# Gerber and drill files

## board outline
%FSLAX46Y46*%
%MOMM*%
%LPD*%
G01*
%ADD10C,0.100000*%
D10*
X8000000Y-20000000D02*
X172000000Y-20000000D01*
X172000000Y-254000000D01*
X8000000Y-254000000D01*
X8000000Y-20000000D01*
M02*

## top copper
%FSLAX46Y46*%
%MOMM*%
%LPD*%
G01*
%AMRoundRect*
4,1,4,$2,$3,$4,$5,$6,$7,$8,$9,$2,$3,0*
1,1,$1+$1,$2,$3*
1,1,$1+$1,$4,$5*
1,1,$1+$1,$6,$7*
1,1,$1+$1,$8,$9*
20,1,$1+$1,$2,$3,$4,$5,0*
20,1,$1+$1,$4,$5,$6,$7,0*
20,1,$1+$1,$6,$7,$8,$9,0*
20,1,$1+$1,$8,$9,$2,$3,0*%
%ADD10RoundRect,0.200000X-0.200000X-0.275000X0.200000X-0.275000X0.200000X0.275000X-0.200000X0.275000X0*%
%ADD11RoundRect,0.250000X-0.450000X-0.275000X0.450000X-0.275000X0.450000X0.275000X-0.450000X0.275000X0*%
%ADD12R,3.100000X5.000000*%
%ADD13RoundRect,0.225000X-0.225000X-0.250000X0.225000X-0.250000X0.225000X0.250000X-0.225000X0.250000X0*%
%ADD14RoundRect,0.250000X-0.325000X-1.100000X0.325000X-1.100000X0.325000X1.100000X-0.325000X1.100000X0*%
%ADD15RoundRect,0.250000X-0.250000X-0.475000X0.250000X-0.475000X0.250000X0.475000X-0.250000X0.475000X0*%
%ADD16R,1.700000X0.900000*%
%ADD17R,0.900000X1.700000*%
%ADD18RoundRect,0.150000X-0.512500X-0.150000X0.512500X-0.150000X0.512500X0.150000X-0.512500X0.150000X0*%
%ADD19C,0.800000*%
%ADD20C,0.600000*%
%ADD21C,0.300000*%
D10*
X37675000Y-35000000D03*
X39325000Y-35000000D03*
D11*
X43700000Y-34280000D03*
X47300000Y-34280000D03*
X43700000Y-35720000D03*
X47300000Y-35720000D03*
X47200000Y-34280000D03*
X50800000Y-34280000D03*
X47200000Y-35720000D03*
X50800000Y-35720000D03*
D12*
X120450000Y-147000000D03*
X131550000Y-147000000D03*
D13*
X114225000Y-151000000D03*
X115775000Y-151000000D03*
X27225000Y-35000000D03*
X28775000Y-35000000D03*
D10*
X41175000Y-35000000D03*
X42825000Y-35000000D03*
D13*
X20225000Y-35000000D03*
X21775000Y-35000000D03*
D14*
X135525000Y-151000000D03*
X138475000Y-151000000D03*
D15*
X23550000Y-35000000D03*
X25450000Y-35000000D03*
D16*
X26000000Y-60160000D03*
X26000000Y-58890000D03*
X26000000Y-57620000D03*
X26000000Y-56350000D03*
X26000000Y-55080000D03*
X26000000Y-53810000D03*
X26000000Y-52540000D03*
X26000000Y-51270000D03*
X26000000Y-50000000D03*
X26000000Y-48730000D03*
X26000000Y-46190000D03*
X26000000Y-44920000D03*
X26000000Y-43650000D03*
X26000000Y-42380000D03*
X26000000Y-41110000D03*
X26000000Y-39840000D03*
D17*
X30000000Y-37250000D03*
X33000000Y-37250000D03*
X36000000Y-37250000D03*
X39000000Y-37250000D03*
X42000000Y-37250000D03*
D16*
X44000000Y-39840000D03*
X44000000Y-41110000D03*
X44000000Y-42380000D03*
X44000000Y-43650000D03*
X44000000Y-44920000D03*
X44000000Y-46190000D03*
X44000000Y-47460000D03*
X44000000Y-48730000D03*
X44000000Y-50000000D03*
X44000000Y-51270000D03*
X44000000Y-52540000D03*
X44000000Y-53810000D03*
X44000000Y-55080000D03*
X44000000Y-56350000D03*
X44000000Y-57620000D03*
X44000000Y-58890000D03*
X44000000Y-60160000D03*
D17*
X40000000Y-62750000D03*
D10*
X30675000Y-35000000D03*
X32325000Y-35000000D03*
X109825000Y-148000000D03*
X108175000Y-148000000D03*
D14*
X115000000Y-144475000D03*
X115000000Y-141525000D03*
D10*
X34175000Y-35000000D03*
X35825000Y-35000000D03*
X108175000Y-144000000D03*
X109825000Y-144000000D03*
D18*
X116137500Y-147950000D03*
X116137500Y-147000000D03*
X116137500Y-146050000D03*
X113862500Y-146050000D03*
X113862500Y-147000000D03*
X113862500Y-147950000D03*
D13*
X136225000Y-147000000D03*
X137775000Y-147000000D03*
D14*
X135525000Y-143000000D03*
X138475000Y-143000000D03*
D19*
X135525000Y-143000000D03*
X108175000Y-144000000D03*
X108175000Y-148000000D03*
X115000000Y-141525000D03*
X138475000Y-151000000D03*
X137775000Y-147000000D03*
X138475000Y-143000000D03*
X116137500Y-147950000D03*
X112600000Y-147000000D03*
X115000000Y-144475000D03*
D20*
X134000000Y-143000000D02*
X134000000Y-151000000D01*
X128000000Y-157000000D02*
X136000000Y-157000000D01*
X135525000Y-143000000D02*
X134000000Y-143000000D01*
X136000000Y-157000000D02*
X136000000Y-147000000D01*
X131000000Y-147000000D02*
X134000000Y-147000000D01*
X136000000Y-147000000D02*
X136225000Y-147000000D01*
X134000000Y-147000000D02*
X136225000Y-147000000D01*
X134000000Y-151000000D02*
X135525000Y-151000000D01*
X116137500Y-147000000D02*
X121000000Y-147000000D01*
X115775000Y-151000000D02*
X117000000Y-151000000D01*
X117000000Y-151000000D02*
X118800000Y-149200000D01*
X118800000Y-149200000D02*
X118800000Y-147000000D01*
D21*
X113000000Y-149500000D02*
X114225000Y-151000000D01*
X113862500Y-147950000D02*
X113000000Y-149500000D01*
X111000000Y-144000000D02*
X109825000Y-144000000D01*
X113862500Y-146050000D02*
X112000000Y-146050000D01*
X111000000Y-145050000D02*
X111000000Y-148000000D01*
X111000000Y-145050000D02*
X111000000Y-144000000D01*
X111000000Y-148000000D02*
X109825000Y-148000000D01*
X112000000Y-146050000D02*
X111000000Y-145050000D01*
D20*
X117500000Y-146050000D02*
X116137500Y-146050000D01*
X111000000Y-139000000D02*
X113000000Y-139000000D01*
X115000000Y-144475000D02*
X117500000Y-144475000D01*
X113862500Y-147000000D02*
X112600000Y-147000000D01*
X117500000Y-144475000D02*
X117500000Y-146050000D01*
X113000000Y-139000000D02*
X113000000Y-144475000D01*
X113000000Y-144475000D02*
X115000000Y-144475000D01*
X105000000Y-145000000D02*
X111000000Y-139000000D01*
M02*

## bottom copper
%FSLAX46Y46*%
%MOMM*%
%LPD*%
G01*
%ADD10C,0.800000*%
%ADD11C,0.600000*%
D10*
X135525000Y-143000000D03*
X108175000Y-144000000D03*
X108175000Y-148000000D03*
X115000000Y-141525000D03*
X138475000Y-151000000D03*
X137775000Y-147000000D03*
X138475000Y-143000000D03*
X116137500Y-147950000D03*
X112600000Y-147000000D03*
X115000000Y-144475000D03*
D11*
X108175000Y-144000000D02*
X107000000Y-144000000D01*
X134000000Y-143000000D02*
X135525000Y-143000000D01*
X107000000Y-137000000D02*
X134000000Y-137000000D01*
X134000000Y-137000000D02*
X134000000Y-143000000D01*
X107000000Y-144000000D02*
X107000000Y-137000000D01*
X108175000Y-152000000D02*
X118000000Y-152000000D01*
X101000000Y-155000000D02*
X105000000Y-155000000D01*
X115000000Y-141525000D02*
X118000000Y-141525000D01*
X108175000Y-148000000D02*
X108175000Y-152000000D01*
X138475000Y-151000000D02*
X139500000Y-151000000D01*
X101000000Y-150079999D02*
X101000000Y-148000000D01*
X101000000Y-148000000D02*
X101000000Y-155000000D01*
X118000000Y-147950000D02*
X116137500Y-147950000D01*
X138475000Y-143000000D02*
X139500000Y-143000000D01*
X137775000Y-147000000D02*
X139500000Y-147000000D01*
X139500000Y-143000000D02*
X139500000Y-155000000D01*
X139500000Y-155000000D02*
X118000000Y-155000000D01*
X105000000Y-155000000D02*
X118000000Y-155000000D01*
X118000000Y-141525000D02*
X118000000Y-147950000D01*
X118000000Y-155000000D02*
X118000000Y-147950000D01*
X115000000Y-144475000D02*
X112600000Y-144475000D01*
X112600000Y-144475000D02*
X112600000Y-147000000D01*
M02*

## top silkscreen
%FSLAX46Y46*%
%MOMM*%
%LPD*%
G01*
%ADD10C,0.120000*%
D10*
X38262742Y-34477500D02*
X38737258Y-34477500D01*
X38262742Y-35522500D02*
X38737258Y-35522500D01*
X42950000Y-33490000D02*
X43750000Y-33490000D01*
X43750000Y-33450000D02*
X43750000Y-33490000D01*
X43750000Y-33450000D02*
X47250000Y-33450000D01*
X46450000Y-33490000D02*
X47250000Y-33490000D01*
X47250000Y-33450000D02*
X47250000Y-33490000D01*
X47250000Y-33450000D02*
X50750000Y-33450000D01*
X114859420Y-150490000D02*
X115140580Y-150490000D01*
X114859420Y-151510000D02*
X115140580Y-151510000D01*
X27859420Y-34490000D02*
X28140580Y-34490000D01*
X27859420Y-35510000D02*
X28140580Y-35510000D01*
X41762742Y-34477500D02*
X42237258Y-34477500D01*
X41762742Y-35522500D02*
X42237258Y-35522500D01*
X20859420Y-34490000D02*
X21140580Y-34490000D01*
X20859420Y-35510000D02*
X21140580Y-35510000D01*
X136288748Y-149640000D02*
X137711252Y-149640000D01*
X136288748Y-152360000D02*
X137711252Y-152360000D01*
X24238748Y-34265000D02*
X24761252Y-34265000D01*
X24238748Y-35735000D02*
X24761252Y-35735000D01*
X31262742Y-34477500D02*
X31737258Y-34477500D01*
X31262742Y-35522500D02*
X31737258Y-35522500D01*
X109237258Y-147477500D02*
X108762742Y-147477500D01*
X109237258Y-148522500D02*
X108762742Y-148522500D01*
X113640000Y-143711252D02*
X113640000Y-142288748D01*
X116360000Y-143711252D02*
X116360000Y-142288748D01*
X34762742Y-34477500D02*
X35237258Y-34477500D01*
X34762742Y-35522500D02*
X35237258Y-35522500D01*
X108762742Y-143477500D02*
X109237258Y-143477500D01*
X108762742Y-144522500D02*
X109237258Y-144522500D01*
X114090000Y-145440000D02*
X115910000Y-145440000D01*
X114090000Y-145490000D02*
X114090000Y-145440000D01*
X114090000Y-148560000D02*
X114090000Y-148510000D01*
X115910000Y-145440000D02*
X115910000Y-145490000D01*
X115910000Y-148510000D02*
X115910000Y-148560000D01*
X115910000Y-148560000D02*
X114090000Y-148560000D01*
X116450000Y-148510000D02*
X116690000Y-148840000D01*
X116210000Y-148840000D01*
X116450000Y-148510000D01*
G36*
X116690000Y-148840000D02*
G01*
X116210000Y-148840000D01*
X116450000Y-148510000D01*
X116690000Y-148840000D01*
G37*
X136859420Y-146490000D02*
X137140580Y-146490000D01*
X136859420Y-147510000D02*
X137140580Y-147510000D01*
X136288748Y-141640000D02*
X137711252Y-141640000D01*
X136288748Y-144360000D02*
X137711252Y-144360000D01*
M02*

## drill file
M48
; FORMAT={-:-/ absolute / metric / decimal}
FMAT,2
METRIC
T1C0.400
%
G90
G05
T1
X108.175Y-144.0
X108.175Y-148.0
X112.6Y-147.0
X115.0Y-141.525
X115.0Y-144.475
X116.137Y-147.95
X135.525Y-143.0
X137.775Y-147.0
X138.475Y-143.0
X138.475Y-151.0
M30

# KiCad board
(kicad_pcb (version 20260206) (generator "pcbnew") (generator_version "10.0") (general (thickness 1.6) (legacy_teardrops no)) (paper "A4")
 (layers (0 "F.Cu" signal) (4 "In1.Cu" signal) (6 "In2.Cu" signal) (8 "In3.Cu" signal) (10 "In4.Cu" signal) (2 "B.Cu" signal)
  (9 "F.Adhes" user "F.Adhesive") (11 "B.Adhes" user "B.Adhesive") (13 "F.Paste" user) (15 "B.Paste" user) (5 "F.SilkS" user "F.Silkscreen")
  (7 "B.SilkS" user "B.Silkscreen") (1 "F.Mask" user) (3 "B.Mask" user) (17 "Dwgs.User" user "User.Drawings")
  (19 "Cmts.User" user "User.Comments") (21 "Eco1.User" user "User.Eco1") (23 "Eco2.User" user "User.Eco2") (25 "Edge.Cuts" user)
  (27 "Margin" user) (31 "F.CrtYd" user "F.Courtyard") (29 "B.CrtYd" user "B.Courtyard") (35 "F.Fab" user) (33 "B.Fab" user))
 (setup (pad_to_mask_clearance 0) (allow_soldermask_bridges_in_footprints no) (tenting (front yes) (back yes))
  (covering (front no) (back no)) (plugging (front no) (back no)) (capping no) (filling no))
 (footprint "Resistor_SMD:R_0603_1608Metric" (layer "F.Cu") (at 38.5 35)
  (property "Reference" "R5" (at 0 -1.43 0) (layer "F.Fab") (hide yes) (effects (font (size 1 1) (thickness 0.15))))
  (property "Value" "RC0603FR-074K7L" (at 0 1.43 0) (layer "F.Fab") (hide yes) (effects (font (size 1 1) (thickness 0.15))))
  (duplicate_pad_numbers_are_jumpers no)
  (fp_line (start -0.237258 -0.5225) (end 0.237258 -0.5225) (stroke (width 0.12) (type solid)) (layer "F.SilkS"))
  (fp_line (start -0.237258 0.5225) (end 0.237258 0.5225) (stroke (width 0.12) (type solid)) (layer "F.SilkS"))
  (pad "1" smd roundrect (at -0.825 0) (size 0.8 0.95) (layers "F.Cu" "F.Mask" "F.Paste") (roundrect_rratio 0.25) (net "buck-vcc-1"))
  (pad "2" smd roundrect (at 0.825 0) (size 0.8 0.95) (layers "F.Cu" "F.Mask" "F.Paste") (roundrect_rratio 0.25) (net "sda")))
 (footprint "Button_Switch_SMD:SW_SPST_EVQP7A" (layer "F.Cu") (at 45.5 35)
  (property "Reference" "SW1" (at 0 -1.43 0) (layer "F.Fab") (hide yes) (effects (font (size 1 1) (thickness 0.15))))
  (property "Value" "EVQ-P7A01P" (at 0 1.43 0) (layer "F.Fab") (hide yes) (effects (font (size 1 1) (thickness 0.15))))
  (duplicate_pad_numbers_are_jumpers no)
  (fp_line (start -2.55 -1.51) (end -1.75 -1.51) (stroke (width 0.12) (type default)) (layer "F.SilkS"))
  (fp_line (start -1.75 -1.55) (end -1.75 -1.51) (stroke (width 0.12) (type default)) (layer "F.SilkS"))
  (fp_line (start -1.75 -1.55) (end 1.75 -1.55) (stroke (width 0.12) (type solid)) (layer "F.SilkS"))
  (pad "1" smd roundrect (at -1.8 -0.72) (size 1.4 1.05) (layers "F.Cu" "F.Mask" "F.Paste") (roundrect_rratio 0.2380952381) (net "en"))
  (pad "1" smd roundrect (at 1.8 -0.72) (size 1.4 1.05) (layers "F.Cu" "F.Mask" "F.Paste") (roundrect_rratio 0.2380952381) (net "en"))
  (pad "2" smd roundrect (at -1.8 0.72) (size 1.4 1.05) (layers "F.Cu" "F.Mask" "F.Paste") (roundrect_rratio 0.2380952381) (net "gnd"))
  (pad "2" smd roundrect (at 1.8 0.72) (size 1.4 1.05) (layers "F.Cu" "F.Mask" "F.Paste") (roundrect_rratio 0.2380952381) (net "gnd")))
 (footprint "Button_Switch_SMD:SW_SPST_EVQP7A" (layer "F.Cu") (at 49 35)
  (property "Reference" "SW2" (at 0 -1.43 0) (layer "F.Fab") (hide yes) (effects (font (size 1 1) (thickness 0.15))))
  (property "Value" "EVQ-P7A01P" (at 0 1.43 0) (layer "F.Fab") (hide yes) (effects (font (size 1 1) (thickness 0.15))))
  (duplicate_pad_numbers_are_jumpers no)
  (fp_line (start -2.55 -1.51) (end -1.75 -1.51) (stroke (width 0.12) (type default)) (layer "F.SilkS"))
  (fp_line (start -1.75 -1.55) (end -1.75 -1.51) (stroke (width 0.12) (type default)) (layer "F.SilkS"))
  (fp_line (start -1.75 -1.55) (end 1.75 -1.55) (stroke (width 0.12) (type solid)) (layer "F.SilkS"))
  (pad "1" smd roundrect (at -1.8 -0.72) (size 1.4 1.05) (layers "F.Cu" "F.Mask" "F.Paste") (roundrect_rratio 0.2380952381) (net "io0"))
  (pad "1" smd roundrect (at 1.8 -0.72) (size 1.4 1.05) (layers "F.Cu" "F.Mask" "F.Paste") (roundrect_rratio 0.2380952381) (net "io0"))
  (pad "2" smd roundrect (at -1.8 0.72) (size 1.4 1.05) (layers "F.Cu" "F.Mask" "F.Paste") (roundrect_rratio 0.2380952381) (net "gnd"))
  (pad "2" smd roundrect (at 1.8 0.72) (size 1.4 1.05) (layers "F.Cu" "F.Mask" "F.Paste") (roundrect_rratio 0.2380952381) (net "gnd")))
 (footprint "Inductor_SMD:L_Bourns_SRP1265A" (layer "F.Cu") (at 126 147)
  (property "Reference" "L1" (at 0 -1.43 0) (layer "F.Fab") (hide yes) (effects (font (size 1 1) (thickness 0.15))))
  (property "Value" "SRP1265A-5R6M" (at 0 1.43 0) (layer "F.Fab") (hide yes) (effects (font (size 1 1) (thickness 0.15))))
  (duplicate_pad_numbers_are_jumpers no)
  (pad "1" smd rect (at -5.55 0) (size 3.1 5) (layers "F.Cu" "F.Mask" "F.Paste") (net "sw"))
  (pad "2" smd rect (at 5.55 0) (size 3.1 5) (layers "F.Cu" "F.Mask" "F.Paste") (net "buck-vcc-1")))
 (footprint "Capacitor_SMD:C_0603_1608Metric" (layer "F.Cu") (at 115 151)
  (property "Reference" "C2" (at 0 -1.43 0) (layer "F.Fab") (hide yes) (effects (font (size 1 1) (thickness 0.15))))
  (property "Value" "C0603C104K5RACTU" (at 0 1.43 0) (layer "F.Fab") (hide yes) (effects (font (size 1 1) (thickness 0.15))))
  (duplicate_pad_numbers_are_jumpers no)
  (fp_line (start -0.14058 -0.51) (end 0.14058 -0.51) (stroke (width 0.12) (type solid)) (layer "F.SilkS"))
  (fp_line (start -0.14058 0.51) (end 0.14058 0.51) (stroke (width 0.12) (type solid)) (layer "F.SilkS"))
  (pad "1" smd roundrect (at -0.775 0) (size 0.9 0.95) (layers "F.Cu" "F.Mask" "F.Paste") (roundrect_rratio 0.25) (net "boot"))
  (pad "2" smd roundrect (at 0.775 0) (size 0.9 0.95) (layers "F.Cu" "F.Mask" "F.Paste") (roundrect_rratio 0.25) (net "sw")))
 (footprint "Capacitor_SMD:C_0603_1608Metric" (layer "F.Cu") (at 28 35)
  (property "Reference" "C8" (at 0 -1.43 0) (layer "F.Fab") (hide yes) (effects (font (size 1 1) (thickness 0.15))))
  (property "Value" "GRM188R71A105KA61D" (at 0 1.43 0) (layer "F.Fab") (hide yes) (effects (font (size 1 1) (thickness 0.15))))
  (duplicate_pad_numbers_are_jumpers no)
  (fp_line (start -0.14058 -0.51) (end 0.14058 -0.51) (stroke (width 0.12) (type solid)) (layer "F.SilkS"))
  (fp_line (start -0.14058 0.51) (end 0.14058 0.51) (stroke (width 0.12) (type solid)) (layer "F.SilkS"))
  (pad "1" smd roundrect (at -0.775 0) (size 0.9 0.95) (layers "F.Cu" "F.Mask" "F.Paste") (roundrect_rratio 0.25) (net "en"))
  (pad "2" smd roundrect (at 0.775 0) (size 0.9 0.95) (layers "F.Cu" "F.Mask" "F.Paste") (roundrect_rratio 0.25) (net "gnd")))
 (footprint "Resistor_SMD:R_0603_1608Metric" (layer "F.Cu") (at 42 35)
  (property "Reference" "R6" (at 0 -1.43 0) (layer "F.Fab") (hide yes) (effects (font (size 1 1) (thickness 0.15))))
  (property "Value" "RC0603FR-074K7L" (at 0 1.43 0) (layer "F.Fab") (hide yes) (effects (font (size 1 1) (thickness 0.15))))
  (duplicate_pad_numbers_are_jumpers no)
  (fp_line (start -0.237258 -0.5225) (end 0.237258 -0.5225) (stroke (width 0.12) (type solid)) (layer "F.SilkS"))
  (fp_line (start -0.237258 0.5225) (end 0.237258 0.5225) (stroke (width 0.12) (type solid)) (layer "F.SilkS"))
  (pad "1" smd roundrect (at -0.825 0) (size 0.8 0.95) (layers "F.Cu" "F.Mask" "F.Paste") (roundrect_rratio 0.25) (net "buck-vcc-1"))
  (pad "2" smd roundrect (at 0.825 0) (size 0.8 0.95) (layers "F.Cu" "F.Mask" "F.Paste") (roundrect_rratio 0.25) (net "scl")))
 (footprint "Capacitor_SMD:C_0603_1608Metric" (layer "F.Cu") (at 21 35)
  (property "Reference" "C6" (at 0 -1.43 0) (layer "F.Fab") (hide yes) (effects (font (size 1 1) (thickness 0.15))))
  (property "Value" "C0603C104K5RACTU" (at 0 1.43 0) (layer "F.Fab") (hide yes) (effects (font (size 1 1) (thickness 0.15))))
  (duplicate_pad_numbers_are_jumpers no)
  (fp_line (start -0.14058 -0.51) (end 0.14058 -0.51) (stroke (width 0.12) (type solid)) (layer "F.SilkS"))
  (fp_line (start -0.14058 0.51) (end 0.14058 0.51) (stroke (width 0.12) (type solid)) (layer "F.SilkS"))
  (pad "1" smd roundrect (at -0.775 0) (size 0.9 0.95) (layers "F.Cu" "F.Mask" "F.Paste") (roundrect_rratio 0.25) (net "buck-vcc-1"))
  (pad "2" smd roundrect (at 0.775 0) (size 0.9 0.95) (layers "F.Cu" "F.Mask" "F.Paste") (roundrect_rratio 0.25) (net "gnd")))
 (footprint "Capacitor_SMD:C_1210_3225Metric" (layer "F.Cu") (at 137 151)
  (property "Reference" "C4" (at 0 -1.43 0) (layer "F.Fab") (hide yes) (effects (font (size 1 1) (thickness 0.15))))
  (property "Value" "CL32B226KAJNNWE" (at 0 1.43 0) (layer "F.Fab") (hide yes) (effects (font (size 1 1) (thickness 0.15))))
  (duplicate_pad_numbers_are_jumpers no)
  (fp_line (start -0.711252 -1.36) (end 0.711252 -1.36) (stroke (width 0.12) (type solid)) (layer "F.SilkS"))
  (fp_line (start -0.711252 1.36) (end 0.711252 1.36) (stroke (width 0.12) (type solid)) (layer "F.SilkS"))
  (pad "1" smd roundrect (at -1.475 0) (size 1.15 2.7) (layers "F.Cu" "F.Mask" "F.Paste") (roundrect_rratio 0.217391) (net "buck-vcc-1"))
  (pad "2" smd roundrect (at 1.475 0) (size 1.15 2.7) (layers "F.Cu" "F.Mask" "F.Paste") (roundrect_rratio 0.217391) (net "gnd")))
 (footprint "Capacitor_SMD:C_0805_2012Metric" (layer "F.Cu") (at 24.5 35)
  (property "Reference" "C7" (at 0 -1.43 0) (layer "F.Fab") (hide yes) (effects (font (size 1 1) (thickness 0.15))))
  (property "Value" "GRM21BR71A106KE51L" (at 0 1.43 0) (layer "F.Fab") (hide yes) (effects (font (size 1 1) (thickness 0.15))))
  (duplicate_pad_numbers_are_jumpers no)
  (fp_line (start -0.261252 -0.735) (end 0.261252 -0.735) (stroke (width 0.12) (type solid)) (layer "F.SilkS"))
  (fp_line (start -0.261252 0.735) (end 0.261252 0.735) (stroke (width 0.12) (type solid)) (layer "F.SilkS"))
  (pad "1" smd roundrect (at -0.95 0) (size 1 1.45) (layers "F.Cu" "F.Mask" "F.Paste") (roundrect_rratio 0.25) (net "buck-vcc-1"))
  (pad "2" smd roundrect (at 0.95 0) (size 1 1.45) (layers "F.Cu" "F.Mask" "F.Paste") (roundrect_rratio 0.25) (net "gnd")))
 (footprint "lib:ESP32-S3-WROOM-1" (layer "F.Cu") (at 35 50)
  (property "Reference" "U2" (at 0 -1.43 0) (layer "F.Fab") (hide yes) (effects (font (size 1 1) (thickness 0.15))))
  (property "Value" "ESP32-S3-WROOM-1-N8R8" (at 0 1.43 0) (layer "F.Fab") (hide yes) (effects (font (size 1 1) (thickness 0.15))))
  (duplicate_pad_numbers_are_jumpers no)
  (pad "1" smd rect (at -9 10.16) (size 1.7 0.9) (layers "F.Cu" "F.Mask" "F.Paste") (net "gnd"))
  (pad "2" smd rect (at -9 8.89) (size 1.7 0.9) (layers "F.Cu" "F.Mask" "F.Paste") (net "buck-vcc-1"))
  (pad "3" smd rect (at -9 7.62) (size 1.7 0.9) (layers "F.Cu" "F.Mask" "F.Paste") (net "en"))
  (pad "4" smd rect (at -9 6.35) (size 1.7 0.9) (layers "F.Cu" "F.Mask" "F.Paste") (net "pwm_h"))
  (pad "5" smd rect (at -9 5.08) (size 1.7 0.9) (layers "F.Cu" "F.Mask" "F.Paste") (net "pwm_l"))
  (pad "6" smd rect (at -9 3.81) (size 1.7 0.9) (layers "F.Cu" "F.Mask" "F.Paste") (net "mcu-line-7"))
  (pad "7" smd rect (at -9 2.54) (size 1.7 0.9) (layers "F.Cu" "F.Mask" "F.Paste") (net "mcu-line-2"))
  (pad "8" smd rect (at -9 1.27) (size 1.7 0.9) (layers "F.Cu" "F.Mask" "F.Paste") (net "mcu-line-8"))
  (pad "9" smd rect (at -9 0) (size 1.7 0.9) (layers "F.Cu" "F.Mask" "F.Paste") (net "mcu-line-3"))
  (pad "10" smd rect (at -9 -1.27) (size 1.7 0.9) (layers "F.Cu" "F.Mask" "F.Paste") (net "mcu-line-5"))
  (pad "11" smd rect (at -9 -3.81) (size 1.7 0.9) (layers "F.Cu" "F.Mask" "F.Paste") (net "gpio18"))
  (pad "12" smd rect (at -9 -5.08) (size 1.7 0.9) (layers "F.Cu" "F.Mask" "F.Paste") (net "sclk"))
  (pad "13" smd rect (at -9 -6.35) (size 1.7 0.9) (layers "F.Cu" "F.Mask" "F.Paste") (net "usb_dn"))
  (pad "14" smd rect (at -9 -7.62) (size 1.7 0.9) (layers "F.Cu" "F.Mask" "F.Paste") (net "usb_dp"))
  (pad "15" smd rect (at -9 -8.89) (size 1.7 0.9) (layers "F.Cu" "F.Mask" "F.Paste") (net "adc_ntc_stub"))
  (pad "16" smd rect (at -9 -10.16) (size 1.7 0.9) (layers "F.Cu" "F.Mask" "F.Paste") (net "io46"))
  (pad "17" smd rect (at -5 -12.75) (size 0.9 1.7) (layers "F.Cu" "F.Mask" "F.Paste") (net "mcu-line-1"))
  (pad "18" smd rect (at -2 -12.75) (size 0.9 1.7) (layers "F.Cu" "F.Mask" "F.Paste") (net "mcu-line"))
  (pad "19" smd rect (at 1 -12.75) (size 0.9 1.7) (layers "F.Cu" "F.Mask" "F.Paste") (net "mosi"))
  (pad "20" smd rect (at 4 -12.75) (size 0.9 1.7) (layers "F.Cu" "F.Mask" "F.Paste") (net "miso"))
  (pad "21" smd rect (at 7 -12.75) (size 0.9 1.7) (layers "F.Cu" "F.Mask" "F.Paste") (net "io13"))
  (pad "22" smd rect (at 9 -10.16) (size 1.7 0.9) (layers "F.Cu" "F.Mask" "F.Paste") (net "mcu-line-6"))
  (pad "23" smd rect (at 9 -8.89) (size 1.7 0.9) (layers "F.Cu" "F.Mask" "F.Paste") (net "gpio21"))
  (pad "24" smd rect (at 9 -7.62) (size 1.7 0.9) (layers "F.Cu" "F.Mask" "F.Paste") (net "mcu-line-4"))
  (pad "25" smd rect (at 9 -6.35) (size 1.7 0.9) (layers "F.Cu" "F.Mask" "F.Paste") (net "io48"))
  (pad "26" smd rect (at 9 -5.08) (size 1.7 0.9) (layers "F.Cu" "F.Mask" "F.Paste") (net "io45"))
  (pad "27" smd rect (at 9 -3.81) (size 1.7 0.9) (layers "F.Cu" "F.Mask" "F.Paste") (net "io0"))
  (pad "28" smd rect (at 9 -2.54) (size 1.7 0.9) (layers "F.Cu" "F.Mask" "F.Paste") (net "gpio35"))
  (pad "29" smd rect (at 9 -1.27) (size 1.7 0.9) (layers "F.Cu" "F.Mask" "F.Paste") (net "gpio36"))
  (pad "30" smd rect (at 9 0) (size 1.7 0.9) (layers "F.Cu" "F.Mask" "F.Paste") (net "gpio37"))
  (pad "31" smd rect (at 9 1.27) (size 1.7 0.9) (layers "F.Cu" "F.Mask" "F.Paste") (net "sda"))
  (pad "32" smd rect (at 9 2.54) (size 1.7 0.9) (layers "F.Cu" "F.Mask" "F.Paste") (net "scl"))
  (pad "33" smd rect (at 9 3.81) (size 1.7 0.9) (layers "F.Cu" "F.Mask" "F.Paste") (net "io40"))
  (pad "34" smd rect (at 9 5.08) (size 1.7 0.9) (layers "F.Cu" "F.Mask" "F.Paste") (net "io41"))
  (pad "35" smd rect (at 9 6.35) (size 1.7 0.9) (layers "F.Cu" "F.Mask" "F.Paste") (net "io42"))
  (pad "36" smd rect (at 9 7.62) (size 1.7 0.9) (layers "F.Cu" "F.Mask" "F.Paste") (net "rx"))
  (pad "37" smd rect (at 9 8.89) (size 1.7 0.9) (layers "F.Cu" "F.Mask" "F.Paste") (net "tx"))
  (pad "38" smd rect (at 9 10.16) (size 1.7 0.9) (layers "F.Cu" "F.Mask" "F.Paste") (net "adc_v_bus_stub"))
  (pad "39" smd rect (at 5 12.75) (size 0.9 1.7) (layers "F.Cu" "F.Mask" "F.Paste") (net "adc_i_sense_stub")))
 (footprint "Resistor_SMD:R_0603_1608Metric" (layer "F.Cu") (at 31.5 35)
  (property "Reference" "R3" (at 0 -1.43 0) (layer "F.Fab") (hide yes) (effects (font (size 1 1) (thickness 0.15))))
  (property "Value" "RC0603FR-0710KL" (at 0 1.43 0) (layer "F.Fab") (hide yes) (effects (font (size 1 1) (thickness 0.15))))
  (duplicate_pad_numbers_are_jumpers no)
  (fp_line (start -0.237258 -0.5225) (end 0.237258 -0.5225) (stroke (width 0.12) (type solid)) (layer "F.SilkS"))
  (fp_line (start -0.237258 0.5225) (end 0.237258 0.5225) (stroke (width 0.12) (type solid)) (layer "F.SilkS"))
  (pad "1" smd roundrect (at -0.825 0) (size 0.8 0.95) (layers "F.Cu" "F.Mask" "F.Paste") (roundrect_rratio 0.25) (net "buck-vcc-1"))
  (pad "2" smd roundrect (at 0.825 0) (size 0.8 0.95) (layers "F.Cu" "F.Mask" "F.Paste") (roundrect_rratio 0.25) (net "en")))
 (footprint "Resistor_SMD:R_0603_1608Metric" (layer "F.Cu") (at 109 148 180)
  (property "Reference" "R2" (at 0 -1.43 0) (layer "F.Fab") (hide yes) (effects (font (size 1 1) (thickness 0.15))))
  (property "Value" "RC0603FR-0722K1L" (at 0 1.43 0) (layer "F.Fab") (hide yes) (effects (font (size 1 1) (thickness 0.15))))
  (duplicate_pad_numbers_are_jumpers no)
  (fp_line (start -0.237258 0.5225) (end 0.237258 0.5225) (stroke (width 0.12) (type solid)) (layer "F.SilkS"))
  (fp_line (start -0.237258 -0.5225) (end 0.237258 -0.5225) (stroke (width 0.12) (type solid)) (layer "F.SilkS"))
  (pad "1" smd roundrect (at -0.825 0) (size 0.8 0.95) (layers "F.Cu" "F.Mask" "F.Paste") (roundrect_rratio 0.25) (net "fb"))
  (pad "2" smd roundrect (at 0.825 0) (size 0.8 0.95) (layers "F.Cu" "F.Mask" "F.Paste") (roundrect_rratio 0.25) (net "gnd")))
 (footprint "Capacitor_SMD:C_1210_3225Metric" (layer "F.Cu") (at 115 143 90)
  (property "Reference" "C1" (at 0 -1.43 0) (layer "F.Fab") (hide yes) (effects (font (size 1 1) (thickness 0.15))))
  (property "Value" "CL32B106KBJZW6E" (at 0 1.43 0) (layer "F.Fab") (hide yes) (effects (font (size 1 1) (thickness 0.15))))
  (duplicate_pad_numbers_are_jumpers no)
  (fp_line (start -0.711252 -1.36) (end 0.711252 -1.36) (stroke (width 0.12) (type solid)) (layer "F.SilkS"))
  (fp_line (start -0.711252 1.36) (end 0.711252 1.36) (stroke (width 0.12) (type solid)) (layer "F.SilkS"))
  (pad "1" smd roundrect (at -1.475 0) (size 1.15 2.7) (layers "F.Cu" "F.Mask" "F.Paste") (roundrect_rratio 0.217391) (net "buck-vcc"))
  (pad "2" smd roundrect (at 1.475 0) (size 1.15 2.7) (layers "F.Cu" "F.Mask" "F.Paste") (roundrect_rratio 0.217391) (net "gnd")))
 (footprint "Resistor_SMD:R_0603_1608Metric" (layer "F.Cu") (at 35 35)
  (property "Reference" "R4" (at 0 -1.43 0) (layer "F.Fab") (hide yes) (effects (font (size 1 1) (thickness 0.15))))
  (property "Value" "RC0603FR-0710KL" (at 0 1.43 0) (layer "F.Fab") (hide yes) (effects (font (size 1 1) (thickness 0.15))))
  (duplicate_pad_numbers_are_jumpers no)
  (fp_line (start -0.237258 -0.5225) (end 0.237258 -0.5225) (stroke (width 0.12) (type solid)) (layer "F.SilkS"))
  (fp_line (start -0.237258 0.5225) (end 0.237258 0.5225) (stroke (width 0.12) (type solid)) (layer "F.SilkS"))
  (pad "1" smd roundrect (at -0.825 0) (size 0.8 0.95) (layers "F.Cu" "F.Mask" "F.Paste") (roundrect_rratio 0.25) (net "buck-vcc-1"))
  (pad "2" smd roundrect (at 0.825 0) (size 0.8 0.95) (layers "F.Cu" "F.Mask" "F.Paste") (roundrect_rratio 0.25) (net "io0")))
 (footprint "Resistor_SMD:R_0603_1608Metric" (layer "F.Cu") (at 109 144)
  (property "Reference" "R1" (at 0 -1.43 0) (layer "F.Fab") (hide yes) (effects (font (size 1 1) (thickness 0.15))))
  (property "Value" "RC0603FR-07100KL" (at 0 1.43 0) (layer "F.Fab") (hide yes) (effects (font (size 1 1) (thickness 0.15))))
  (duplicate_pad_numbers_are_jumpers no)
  (fp_line (start -0.237258 -0.5225) (end 0.237258 -0.5225) (stroke (width 0.12) (type solid)) (layer "F.SilkS"))
  (fp_line (start -0.237258 0.5225) (end 0.237258 0.5225) (stroke (width 0.12) (type solid)) (layer "F.SilkS"))
  (pad "1" smd roundrect (at -0.825 0) (size 0.8 0.95) (layers "F.Cu" "F.Mask" "F.Paste") (roundrect_rratio 0.25) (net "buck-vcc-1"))
  (pad "2" smd roundrect (at 0.825 0) (size 0.8 0.95) (layers "F.Cu" "F.Mask" "F.Paste") (roundrect_rratio 0.25) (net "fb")))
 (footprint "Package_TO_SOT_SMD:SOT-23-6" (layer "F.Cu") (at 115 147 180)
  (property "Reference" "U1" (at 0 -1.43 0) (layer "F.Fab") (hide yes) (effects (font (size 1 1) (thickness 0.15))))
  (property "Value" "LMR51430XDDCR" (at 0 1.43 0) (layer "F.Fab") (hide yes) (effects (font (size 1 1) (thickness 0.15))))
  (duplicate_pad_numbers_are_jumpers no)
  (fp_line (start 0.91 1.56) (end -0.91 1.56) (stroke (width 0.12) (type solid)) (layer "F.SilkS"))
  (fp_line (start 0.91 1.51) (end 0.91 1.56) (stroke (width 0.12) (type solid)) (layer "F.SilkS"))
  (fp_line (start 0.91 -1.56) (end 0.91 -1.51) (stroke (width 0.12) (type solid)) (layer "F.SilkS"))
  (fp_line (start -0.91 1.56) (end -0.91 1.51) (stroke (width 0.12) (type solid)) (layer "F.SilkS"))
  (fp_line (start -0.91 -1.51) (end -0.91 -1.56) (stroke (width 0.12) (type solid)) (layer "F.SilkS"))
  (fp_line (start -0.91 -1.56) (end 0.91 -1.56) (stroke (width 0.12) (type solid)) (layer "F.SilkS"))
  (fp_poly (pts (xy -1.45 -1.51) (xy -1.69 -1.84) (xy -1.21 -1.84)) (stroke (width 0.12) (type solid)) (fill yes) (layer "F.SilkS"))
  (pad "1" smd roundrect (at -1.1375 -0.95) (size 1.325 0.6) (layers "F.Cu" "F.Mask" "F.Paste") (roundrect_rratio 0.25) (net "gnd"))
  (pad "2" smd roundrect (at -1.1375 0) (size 1.325 0.6) (layers "F.Cu" "F.Mask" "F.Paste") (roundrect_rratio 0.25) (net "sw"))
  (pad "3" smd roundrect (at -1.1375 0.95) (size 1.325 0.6) (layers "F.Cu" "F.Mask" "F.Paste") (roundrect_rratio 0.25) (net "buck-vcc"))
  (pad "4" smd roundrect (at 1.1375 0.95) (size 1.325 0.6) (layers "F.Cu" "F.Mask" "F.Paste") (roundrect_rratio 0.25) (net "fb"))
  (pad "5" smd roundrect (at 1.1375 0) (size 1.325 0.6) (layers "F.Cu" "F.Mask" "F.Paste") (roundrect_rratio 0.25) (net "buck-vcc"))
  (pad "6" smd roundrect (at 1.1375 -0.95) (size 1.325 0.6) (layers "F.Cu" "F.Mask" "F.Paste") (roundrect_rratio 0.25) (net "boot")))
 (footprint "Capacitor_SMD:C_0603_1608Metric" (layer "F.Cu") (at 137 147)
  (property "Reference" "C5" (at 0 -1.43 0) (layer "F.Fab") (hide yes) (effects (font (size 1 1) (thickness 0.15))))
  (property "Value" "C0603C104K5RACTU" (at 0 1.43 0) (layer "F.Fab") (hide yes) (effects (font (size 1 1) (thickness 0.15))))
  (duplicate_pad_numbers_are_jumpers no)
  (fp_line (start -0.14058 -0.51) (end 0.14058 -0.51) (stroke (width 0.12) (type solid)) (layer "F.SilkS"))
  (fp_line (start -0.14058 0.51) (end 0.14058 0.51) (stroke (width 0.12) (type solid)) (layer "F.SilkS"))
  (pad "1" smd roundrect (at -0.775 0) (size 0.9 0.95) (layers "F.Cu" "F.Mask" "F.Paste") (roundrect_rratio 0.25) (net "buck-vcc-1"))
  (pad "2" smd roundrect (at 0.775 0) (size 0.9 0.95) (layers "F.Cu" "F.Mask" "F.Paste") (roundrect_rratio 0.25) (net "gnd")))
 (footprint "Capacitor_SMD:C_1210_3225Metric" (layer "F.Cu") (at 137 143)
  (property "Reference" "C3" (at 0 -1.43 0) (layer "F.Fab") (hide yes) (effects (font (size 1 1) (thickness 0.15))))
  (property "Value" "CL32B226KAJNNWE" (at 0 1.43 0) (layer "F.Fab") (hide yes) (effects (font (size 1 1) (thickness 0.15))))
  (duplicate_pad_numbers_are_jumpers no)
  (fp_line (start -0.711252 -1.36) (end 0.711252 -1.36) (stroke (width 0.12) (type solid)) (layer "F.SilkS"))
  (fp_line (start -0.711252 1.36) (end 0.711252 1.36) (stroke (width 0.12) (type solid)) (layer "F.SilkS"))
  (pad "1" smd roundrect (at -1.475 0) (size 1.15 2.7) (layers "F.Cu" "F.Mask" "F.Paste") (roundrect_rratio 0.217391) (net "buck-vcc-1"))
  (pad "2" smd roundrect (at 1.475 0) (size 1.15 2.7) (layers "F.Cu" "F.Mask" "F.Paste") (roundrect_rratio 0.217391) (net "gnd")))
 (gr_poly (pts (xy 8 20) (xy 172 20) (xy 172 254) (xy 8 254)) (stroke (width 0.1) (type solid)) (fill no) (layer "Edge.Cuts"))
 (segment (start 134 143) (end 134 151) (width 0.6) (layer "F.Cu") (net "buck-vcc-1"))
 (segment (start 128 157) (end 136 157) (width 0.6) (layer "F.Cu") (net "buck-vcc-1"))
 (segment (start 135.525 143) (end 134 143) (width 0.6) (layer "F.Cu") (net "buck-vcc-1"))
 (segment (start 136 157) (end 136 147) (width 0.6) (layer "F.Cu") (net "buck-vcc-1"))
 (segment (start 131 147) (end 134 147) (width 0.6) (layer "F.Cu") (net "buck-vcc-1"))
 (segment (start 136 147) (end 136.225 147) (width 0.6) (layer "F.Cu") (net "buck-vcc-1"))
 (segment (start 134 147) (end 136.225 147) (width 0.6) (layer "F.Cu") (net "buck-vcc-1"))
 (segment (start 134 151) (end 135.525 151) (width 0.6) (layer "F.Cu") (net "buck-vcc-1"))
 (via (at 135.525 143) (size 0.8) (drill 0.4) (layers "F.Cu" "B.Cu") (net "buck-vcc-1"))
 (via (at 108.175 144) (size 0.8) (drill 0.4) (layers "F.Cu" "B.Cu") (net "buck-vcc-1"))
 (segment (start 108.175 144) (end 107 144) (width 0.6) (layer "B.Cu") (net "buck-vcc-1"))
 (segment (start 134 143) (end 135.525 143) (width 0.6) (layer "B.Cu") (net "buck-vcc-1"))
 (segment (start 107 137) (end 134 137) (width 0.6) (layer "B.Cu") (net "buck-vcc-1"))
 (segment (start 134 137) (end 134 143) (width 0.6) (layer "B.Cu") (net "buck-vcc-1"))
 (segment (start 107 144) (end 107 137) (width 0.6) (layer "B.Cu") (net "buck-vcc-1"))
 (via (at 108.175 148) (size 0.8) (drill 0.4) (layers "F.Cu" "B.Cu") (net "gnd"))
 (via (at 115 141.525) (size 0.8) (drill 0.4) (layers "F.Cu" "B.Cu") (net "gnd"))
 (via (at 138.475 151) (size 0.8) (drill 0.4) (layers "F.Cu" "B.Cu") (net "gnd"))
 (via (at 137.775 147) (size 0.8) (drill 0.4) (layers "F.Cu" "B.Cu") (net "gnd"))
 (via (at 138.475 143) (size 0.8) (drill 0.4) (layers "F.Cu" "B.Cu") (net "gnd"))
 (via (at 116.1375 147.95) (size 0.8) (drill 0.4) (layers "F.Cu" "B.Cu") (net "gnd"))
 (segment (start 108.175 152) (end 118 152) (width 0.6) (layer "B.Cu") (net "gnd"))
 (segment (start 101 155) (end 105 155) (width 0.6) (layer "B.Cu") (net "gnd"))
 (segment (start 115 141.525) (end 118 141.525) (width 0.6) (layer "B.Cu") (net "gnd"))
 (segment (start 108.175 148) (end 108.175 152) (width 0.6) (layer "B.Cu") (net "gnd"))
 (segment (start 138.475 151) (end 139.5 151) (width 0.6) (layer "B.Cu") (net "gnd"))
 (segment (start 101 150.079999) (end 101 148) (width 0.6) (layer "B.Cu") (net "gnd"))
 (segment (start 101 148) (end 101 155) (width 0.6) (layer "B.Cu") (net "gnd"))
 (segment (start 118 147.95) (end 116.1375 147.95) (width 0.6) (layer "B.Cu") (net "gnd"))
 (segment (start 138.475 143) (end 139.5 143) (width 0.6) (layer "B.Cu") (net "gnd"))
 (segment (start 137.775 147) (end 139.5 147) (width 0.6) (layer "B.Cu") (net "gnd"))
 (segment (start 139.5 143) (end 139.5 155) (width 0.6) (layer "B.Cu") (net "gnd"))
 (segment (start 139.5 155) (end 118 155) (width 0.6) (layer "B.Cu") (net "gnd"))
 (segment (start 105 155) (end 118 155) (width 0.6) (layer "B.Cu") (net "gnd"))
 (segment (start 118 141.525) (end 118 147.95) (width 0.6) (layer "B.Cu") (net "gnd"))
 (segment (start 118 155) (end 118 147.95) (width 0.6) (layer "B.Cu") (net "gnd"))
 (segment (start 116.1375 147) (end 121 147) (width 0.6) (layer "F.Cu") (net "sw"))
 (segment (start 115.775 151) (end 117 151) (width 0.6) (layer "F.Cu") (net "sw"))
 (segment (start 117 151) (end 118.8 149.2) (width 0.6) (layer "F.Cu") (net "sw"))
 (segment (start 118.8 149.2) (end 118.8 147) (width 0.6) (layer "F.Cu") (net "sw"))
 (segment (start 113 149.5) (end 114.225 151) (width 0.3) (layer "F.Cu") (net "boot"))
 (segment (start 113.8625 147.95) (end 113 149.5) (width 0.3) (layer "F.Cu") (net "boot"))
 (segment (start 111 144) (end 109.825 144) (width 0.3) (layer "F.Cu") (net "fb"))
 (segment (start 113.8625 146.05) (end 112 146.05) (width 0.3) (layer "F.Cu") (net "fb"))
 (segment (start 111 145.05) (end 111 148) (width 0.3) (layer "F.Cu") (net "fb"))
 (segment (start 111 145.05) (end 111 144) (width 0.3) (layer "F.Cu") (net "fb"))
 (segment (start 111 148) (end 109.825 148) (width 0.3) (layer "F.Cu") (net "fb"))
 (segment (start 112 146.05) (end 111 145.05) (width 0.3) (layer "F.Cu") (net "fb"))
 (segment (start 117.5 146.05) (end 116.1375 146.05) (width 0.6) (layer "F.Cu") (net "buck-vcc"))
 (segment (start 111 139) (end 113 139) (width 0.6) (layer "F.Cu") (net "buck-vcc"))
 (segment (start 115 144.475) (end 117.5 144.475) (width 0.6) (layer "F.Cu") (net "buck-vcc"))
 (segment (start 113.8625 147) (end 112.6 147) (width 0.6) (layer "F.Cu") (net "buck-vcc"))
 (segment (start 117.5 144.475) (end 117.5 146.05) (width 0.6) (layer "F.Cu") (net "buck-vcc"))
 (segment (start 113 139) (end 113 144.475) (width 0.6) (layer "F.Cu") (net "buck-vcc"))
 (segment (start 113 144.475) (end 115 144.475) (width 0.6) (layer "F.Cu") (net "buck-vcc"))
 (segment (start 105 145) (end 111 139) (width 0.6) (layer "F.Cu") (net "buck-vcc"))
 (via (at 112.6 147) (size 0.8) (drill 0.4) (layers "F.Cu" "B.Cu") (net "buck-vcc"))
 (via (at 115 144.475) (size 0.8) (drill 0.4) (layers "F.Cu" "B.Cu") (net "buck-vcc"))
 (segment (start 115 144.475) (end 112.6 144.475) (width 0.6) (layer "B.Cu") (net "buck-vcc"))
 (segment (start 112.6 144.475) (end 112.6 147) (width 0.6) (layer "B.Cu") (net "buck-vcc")))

